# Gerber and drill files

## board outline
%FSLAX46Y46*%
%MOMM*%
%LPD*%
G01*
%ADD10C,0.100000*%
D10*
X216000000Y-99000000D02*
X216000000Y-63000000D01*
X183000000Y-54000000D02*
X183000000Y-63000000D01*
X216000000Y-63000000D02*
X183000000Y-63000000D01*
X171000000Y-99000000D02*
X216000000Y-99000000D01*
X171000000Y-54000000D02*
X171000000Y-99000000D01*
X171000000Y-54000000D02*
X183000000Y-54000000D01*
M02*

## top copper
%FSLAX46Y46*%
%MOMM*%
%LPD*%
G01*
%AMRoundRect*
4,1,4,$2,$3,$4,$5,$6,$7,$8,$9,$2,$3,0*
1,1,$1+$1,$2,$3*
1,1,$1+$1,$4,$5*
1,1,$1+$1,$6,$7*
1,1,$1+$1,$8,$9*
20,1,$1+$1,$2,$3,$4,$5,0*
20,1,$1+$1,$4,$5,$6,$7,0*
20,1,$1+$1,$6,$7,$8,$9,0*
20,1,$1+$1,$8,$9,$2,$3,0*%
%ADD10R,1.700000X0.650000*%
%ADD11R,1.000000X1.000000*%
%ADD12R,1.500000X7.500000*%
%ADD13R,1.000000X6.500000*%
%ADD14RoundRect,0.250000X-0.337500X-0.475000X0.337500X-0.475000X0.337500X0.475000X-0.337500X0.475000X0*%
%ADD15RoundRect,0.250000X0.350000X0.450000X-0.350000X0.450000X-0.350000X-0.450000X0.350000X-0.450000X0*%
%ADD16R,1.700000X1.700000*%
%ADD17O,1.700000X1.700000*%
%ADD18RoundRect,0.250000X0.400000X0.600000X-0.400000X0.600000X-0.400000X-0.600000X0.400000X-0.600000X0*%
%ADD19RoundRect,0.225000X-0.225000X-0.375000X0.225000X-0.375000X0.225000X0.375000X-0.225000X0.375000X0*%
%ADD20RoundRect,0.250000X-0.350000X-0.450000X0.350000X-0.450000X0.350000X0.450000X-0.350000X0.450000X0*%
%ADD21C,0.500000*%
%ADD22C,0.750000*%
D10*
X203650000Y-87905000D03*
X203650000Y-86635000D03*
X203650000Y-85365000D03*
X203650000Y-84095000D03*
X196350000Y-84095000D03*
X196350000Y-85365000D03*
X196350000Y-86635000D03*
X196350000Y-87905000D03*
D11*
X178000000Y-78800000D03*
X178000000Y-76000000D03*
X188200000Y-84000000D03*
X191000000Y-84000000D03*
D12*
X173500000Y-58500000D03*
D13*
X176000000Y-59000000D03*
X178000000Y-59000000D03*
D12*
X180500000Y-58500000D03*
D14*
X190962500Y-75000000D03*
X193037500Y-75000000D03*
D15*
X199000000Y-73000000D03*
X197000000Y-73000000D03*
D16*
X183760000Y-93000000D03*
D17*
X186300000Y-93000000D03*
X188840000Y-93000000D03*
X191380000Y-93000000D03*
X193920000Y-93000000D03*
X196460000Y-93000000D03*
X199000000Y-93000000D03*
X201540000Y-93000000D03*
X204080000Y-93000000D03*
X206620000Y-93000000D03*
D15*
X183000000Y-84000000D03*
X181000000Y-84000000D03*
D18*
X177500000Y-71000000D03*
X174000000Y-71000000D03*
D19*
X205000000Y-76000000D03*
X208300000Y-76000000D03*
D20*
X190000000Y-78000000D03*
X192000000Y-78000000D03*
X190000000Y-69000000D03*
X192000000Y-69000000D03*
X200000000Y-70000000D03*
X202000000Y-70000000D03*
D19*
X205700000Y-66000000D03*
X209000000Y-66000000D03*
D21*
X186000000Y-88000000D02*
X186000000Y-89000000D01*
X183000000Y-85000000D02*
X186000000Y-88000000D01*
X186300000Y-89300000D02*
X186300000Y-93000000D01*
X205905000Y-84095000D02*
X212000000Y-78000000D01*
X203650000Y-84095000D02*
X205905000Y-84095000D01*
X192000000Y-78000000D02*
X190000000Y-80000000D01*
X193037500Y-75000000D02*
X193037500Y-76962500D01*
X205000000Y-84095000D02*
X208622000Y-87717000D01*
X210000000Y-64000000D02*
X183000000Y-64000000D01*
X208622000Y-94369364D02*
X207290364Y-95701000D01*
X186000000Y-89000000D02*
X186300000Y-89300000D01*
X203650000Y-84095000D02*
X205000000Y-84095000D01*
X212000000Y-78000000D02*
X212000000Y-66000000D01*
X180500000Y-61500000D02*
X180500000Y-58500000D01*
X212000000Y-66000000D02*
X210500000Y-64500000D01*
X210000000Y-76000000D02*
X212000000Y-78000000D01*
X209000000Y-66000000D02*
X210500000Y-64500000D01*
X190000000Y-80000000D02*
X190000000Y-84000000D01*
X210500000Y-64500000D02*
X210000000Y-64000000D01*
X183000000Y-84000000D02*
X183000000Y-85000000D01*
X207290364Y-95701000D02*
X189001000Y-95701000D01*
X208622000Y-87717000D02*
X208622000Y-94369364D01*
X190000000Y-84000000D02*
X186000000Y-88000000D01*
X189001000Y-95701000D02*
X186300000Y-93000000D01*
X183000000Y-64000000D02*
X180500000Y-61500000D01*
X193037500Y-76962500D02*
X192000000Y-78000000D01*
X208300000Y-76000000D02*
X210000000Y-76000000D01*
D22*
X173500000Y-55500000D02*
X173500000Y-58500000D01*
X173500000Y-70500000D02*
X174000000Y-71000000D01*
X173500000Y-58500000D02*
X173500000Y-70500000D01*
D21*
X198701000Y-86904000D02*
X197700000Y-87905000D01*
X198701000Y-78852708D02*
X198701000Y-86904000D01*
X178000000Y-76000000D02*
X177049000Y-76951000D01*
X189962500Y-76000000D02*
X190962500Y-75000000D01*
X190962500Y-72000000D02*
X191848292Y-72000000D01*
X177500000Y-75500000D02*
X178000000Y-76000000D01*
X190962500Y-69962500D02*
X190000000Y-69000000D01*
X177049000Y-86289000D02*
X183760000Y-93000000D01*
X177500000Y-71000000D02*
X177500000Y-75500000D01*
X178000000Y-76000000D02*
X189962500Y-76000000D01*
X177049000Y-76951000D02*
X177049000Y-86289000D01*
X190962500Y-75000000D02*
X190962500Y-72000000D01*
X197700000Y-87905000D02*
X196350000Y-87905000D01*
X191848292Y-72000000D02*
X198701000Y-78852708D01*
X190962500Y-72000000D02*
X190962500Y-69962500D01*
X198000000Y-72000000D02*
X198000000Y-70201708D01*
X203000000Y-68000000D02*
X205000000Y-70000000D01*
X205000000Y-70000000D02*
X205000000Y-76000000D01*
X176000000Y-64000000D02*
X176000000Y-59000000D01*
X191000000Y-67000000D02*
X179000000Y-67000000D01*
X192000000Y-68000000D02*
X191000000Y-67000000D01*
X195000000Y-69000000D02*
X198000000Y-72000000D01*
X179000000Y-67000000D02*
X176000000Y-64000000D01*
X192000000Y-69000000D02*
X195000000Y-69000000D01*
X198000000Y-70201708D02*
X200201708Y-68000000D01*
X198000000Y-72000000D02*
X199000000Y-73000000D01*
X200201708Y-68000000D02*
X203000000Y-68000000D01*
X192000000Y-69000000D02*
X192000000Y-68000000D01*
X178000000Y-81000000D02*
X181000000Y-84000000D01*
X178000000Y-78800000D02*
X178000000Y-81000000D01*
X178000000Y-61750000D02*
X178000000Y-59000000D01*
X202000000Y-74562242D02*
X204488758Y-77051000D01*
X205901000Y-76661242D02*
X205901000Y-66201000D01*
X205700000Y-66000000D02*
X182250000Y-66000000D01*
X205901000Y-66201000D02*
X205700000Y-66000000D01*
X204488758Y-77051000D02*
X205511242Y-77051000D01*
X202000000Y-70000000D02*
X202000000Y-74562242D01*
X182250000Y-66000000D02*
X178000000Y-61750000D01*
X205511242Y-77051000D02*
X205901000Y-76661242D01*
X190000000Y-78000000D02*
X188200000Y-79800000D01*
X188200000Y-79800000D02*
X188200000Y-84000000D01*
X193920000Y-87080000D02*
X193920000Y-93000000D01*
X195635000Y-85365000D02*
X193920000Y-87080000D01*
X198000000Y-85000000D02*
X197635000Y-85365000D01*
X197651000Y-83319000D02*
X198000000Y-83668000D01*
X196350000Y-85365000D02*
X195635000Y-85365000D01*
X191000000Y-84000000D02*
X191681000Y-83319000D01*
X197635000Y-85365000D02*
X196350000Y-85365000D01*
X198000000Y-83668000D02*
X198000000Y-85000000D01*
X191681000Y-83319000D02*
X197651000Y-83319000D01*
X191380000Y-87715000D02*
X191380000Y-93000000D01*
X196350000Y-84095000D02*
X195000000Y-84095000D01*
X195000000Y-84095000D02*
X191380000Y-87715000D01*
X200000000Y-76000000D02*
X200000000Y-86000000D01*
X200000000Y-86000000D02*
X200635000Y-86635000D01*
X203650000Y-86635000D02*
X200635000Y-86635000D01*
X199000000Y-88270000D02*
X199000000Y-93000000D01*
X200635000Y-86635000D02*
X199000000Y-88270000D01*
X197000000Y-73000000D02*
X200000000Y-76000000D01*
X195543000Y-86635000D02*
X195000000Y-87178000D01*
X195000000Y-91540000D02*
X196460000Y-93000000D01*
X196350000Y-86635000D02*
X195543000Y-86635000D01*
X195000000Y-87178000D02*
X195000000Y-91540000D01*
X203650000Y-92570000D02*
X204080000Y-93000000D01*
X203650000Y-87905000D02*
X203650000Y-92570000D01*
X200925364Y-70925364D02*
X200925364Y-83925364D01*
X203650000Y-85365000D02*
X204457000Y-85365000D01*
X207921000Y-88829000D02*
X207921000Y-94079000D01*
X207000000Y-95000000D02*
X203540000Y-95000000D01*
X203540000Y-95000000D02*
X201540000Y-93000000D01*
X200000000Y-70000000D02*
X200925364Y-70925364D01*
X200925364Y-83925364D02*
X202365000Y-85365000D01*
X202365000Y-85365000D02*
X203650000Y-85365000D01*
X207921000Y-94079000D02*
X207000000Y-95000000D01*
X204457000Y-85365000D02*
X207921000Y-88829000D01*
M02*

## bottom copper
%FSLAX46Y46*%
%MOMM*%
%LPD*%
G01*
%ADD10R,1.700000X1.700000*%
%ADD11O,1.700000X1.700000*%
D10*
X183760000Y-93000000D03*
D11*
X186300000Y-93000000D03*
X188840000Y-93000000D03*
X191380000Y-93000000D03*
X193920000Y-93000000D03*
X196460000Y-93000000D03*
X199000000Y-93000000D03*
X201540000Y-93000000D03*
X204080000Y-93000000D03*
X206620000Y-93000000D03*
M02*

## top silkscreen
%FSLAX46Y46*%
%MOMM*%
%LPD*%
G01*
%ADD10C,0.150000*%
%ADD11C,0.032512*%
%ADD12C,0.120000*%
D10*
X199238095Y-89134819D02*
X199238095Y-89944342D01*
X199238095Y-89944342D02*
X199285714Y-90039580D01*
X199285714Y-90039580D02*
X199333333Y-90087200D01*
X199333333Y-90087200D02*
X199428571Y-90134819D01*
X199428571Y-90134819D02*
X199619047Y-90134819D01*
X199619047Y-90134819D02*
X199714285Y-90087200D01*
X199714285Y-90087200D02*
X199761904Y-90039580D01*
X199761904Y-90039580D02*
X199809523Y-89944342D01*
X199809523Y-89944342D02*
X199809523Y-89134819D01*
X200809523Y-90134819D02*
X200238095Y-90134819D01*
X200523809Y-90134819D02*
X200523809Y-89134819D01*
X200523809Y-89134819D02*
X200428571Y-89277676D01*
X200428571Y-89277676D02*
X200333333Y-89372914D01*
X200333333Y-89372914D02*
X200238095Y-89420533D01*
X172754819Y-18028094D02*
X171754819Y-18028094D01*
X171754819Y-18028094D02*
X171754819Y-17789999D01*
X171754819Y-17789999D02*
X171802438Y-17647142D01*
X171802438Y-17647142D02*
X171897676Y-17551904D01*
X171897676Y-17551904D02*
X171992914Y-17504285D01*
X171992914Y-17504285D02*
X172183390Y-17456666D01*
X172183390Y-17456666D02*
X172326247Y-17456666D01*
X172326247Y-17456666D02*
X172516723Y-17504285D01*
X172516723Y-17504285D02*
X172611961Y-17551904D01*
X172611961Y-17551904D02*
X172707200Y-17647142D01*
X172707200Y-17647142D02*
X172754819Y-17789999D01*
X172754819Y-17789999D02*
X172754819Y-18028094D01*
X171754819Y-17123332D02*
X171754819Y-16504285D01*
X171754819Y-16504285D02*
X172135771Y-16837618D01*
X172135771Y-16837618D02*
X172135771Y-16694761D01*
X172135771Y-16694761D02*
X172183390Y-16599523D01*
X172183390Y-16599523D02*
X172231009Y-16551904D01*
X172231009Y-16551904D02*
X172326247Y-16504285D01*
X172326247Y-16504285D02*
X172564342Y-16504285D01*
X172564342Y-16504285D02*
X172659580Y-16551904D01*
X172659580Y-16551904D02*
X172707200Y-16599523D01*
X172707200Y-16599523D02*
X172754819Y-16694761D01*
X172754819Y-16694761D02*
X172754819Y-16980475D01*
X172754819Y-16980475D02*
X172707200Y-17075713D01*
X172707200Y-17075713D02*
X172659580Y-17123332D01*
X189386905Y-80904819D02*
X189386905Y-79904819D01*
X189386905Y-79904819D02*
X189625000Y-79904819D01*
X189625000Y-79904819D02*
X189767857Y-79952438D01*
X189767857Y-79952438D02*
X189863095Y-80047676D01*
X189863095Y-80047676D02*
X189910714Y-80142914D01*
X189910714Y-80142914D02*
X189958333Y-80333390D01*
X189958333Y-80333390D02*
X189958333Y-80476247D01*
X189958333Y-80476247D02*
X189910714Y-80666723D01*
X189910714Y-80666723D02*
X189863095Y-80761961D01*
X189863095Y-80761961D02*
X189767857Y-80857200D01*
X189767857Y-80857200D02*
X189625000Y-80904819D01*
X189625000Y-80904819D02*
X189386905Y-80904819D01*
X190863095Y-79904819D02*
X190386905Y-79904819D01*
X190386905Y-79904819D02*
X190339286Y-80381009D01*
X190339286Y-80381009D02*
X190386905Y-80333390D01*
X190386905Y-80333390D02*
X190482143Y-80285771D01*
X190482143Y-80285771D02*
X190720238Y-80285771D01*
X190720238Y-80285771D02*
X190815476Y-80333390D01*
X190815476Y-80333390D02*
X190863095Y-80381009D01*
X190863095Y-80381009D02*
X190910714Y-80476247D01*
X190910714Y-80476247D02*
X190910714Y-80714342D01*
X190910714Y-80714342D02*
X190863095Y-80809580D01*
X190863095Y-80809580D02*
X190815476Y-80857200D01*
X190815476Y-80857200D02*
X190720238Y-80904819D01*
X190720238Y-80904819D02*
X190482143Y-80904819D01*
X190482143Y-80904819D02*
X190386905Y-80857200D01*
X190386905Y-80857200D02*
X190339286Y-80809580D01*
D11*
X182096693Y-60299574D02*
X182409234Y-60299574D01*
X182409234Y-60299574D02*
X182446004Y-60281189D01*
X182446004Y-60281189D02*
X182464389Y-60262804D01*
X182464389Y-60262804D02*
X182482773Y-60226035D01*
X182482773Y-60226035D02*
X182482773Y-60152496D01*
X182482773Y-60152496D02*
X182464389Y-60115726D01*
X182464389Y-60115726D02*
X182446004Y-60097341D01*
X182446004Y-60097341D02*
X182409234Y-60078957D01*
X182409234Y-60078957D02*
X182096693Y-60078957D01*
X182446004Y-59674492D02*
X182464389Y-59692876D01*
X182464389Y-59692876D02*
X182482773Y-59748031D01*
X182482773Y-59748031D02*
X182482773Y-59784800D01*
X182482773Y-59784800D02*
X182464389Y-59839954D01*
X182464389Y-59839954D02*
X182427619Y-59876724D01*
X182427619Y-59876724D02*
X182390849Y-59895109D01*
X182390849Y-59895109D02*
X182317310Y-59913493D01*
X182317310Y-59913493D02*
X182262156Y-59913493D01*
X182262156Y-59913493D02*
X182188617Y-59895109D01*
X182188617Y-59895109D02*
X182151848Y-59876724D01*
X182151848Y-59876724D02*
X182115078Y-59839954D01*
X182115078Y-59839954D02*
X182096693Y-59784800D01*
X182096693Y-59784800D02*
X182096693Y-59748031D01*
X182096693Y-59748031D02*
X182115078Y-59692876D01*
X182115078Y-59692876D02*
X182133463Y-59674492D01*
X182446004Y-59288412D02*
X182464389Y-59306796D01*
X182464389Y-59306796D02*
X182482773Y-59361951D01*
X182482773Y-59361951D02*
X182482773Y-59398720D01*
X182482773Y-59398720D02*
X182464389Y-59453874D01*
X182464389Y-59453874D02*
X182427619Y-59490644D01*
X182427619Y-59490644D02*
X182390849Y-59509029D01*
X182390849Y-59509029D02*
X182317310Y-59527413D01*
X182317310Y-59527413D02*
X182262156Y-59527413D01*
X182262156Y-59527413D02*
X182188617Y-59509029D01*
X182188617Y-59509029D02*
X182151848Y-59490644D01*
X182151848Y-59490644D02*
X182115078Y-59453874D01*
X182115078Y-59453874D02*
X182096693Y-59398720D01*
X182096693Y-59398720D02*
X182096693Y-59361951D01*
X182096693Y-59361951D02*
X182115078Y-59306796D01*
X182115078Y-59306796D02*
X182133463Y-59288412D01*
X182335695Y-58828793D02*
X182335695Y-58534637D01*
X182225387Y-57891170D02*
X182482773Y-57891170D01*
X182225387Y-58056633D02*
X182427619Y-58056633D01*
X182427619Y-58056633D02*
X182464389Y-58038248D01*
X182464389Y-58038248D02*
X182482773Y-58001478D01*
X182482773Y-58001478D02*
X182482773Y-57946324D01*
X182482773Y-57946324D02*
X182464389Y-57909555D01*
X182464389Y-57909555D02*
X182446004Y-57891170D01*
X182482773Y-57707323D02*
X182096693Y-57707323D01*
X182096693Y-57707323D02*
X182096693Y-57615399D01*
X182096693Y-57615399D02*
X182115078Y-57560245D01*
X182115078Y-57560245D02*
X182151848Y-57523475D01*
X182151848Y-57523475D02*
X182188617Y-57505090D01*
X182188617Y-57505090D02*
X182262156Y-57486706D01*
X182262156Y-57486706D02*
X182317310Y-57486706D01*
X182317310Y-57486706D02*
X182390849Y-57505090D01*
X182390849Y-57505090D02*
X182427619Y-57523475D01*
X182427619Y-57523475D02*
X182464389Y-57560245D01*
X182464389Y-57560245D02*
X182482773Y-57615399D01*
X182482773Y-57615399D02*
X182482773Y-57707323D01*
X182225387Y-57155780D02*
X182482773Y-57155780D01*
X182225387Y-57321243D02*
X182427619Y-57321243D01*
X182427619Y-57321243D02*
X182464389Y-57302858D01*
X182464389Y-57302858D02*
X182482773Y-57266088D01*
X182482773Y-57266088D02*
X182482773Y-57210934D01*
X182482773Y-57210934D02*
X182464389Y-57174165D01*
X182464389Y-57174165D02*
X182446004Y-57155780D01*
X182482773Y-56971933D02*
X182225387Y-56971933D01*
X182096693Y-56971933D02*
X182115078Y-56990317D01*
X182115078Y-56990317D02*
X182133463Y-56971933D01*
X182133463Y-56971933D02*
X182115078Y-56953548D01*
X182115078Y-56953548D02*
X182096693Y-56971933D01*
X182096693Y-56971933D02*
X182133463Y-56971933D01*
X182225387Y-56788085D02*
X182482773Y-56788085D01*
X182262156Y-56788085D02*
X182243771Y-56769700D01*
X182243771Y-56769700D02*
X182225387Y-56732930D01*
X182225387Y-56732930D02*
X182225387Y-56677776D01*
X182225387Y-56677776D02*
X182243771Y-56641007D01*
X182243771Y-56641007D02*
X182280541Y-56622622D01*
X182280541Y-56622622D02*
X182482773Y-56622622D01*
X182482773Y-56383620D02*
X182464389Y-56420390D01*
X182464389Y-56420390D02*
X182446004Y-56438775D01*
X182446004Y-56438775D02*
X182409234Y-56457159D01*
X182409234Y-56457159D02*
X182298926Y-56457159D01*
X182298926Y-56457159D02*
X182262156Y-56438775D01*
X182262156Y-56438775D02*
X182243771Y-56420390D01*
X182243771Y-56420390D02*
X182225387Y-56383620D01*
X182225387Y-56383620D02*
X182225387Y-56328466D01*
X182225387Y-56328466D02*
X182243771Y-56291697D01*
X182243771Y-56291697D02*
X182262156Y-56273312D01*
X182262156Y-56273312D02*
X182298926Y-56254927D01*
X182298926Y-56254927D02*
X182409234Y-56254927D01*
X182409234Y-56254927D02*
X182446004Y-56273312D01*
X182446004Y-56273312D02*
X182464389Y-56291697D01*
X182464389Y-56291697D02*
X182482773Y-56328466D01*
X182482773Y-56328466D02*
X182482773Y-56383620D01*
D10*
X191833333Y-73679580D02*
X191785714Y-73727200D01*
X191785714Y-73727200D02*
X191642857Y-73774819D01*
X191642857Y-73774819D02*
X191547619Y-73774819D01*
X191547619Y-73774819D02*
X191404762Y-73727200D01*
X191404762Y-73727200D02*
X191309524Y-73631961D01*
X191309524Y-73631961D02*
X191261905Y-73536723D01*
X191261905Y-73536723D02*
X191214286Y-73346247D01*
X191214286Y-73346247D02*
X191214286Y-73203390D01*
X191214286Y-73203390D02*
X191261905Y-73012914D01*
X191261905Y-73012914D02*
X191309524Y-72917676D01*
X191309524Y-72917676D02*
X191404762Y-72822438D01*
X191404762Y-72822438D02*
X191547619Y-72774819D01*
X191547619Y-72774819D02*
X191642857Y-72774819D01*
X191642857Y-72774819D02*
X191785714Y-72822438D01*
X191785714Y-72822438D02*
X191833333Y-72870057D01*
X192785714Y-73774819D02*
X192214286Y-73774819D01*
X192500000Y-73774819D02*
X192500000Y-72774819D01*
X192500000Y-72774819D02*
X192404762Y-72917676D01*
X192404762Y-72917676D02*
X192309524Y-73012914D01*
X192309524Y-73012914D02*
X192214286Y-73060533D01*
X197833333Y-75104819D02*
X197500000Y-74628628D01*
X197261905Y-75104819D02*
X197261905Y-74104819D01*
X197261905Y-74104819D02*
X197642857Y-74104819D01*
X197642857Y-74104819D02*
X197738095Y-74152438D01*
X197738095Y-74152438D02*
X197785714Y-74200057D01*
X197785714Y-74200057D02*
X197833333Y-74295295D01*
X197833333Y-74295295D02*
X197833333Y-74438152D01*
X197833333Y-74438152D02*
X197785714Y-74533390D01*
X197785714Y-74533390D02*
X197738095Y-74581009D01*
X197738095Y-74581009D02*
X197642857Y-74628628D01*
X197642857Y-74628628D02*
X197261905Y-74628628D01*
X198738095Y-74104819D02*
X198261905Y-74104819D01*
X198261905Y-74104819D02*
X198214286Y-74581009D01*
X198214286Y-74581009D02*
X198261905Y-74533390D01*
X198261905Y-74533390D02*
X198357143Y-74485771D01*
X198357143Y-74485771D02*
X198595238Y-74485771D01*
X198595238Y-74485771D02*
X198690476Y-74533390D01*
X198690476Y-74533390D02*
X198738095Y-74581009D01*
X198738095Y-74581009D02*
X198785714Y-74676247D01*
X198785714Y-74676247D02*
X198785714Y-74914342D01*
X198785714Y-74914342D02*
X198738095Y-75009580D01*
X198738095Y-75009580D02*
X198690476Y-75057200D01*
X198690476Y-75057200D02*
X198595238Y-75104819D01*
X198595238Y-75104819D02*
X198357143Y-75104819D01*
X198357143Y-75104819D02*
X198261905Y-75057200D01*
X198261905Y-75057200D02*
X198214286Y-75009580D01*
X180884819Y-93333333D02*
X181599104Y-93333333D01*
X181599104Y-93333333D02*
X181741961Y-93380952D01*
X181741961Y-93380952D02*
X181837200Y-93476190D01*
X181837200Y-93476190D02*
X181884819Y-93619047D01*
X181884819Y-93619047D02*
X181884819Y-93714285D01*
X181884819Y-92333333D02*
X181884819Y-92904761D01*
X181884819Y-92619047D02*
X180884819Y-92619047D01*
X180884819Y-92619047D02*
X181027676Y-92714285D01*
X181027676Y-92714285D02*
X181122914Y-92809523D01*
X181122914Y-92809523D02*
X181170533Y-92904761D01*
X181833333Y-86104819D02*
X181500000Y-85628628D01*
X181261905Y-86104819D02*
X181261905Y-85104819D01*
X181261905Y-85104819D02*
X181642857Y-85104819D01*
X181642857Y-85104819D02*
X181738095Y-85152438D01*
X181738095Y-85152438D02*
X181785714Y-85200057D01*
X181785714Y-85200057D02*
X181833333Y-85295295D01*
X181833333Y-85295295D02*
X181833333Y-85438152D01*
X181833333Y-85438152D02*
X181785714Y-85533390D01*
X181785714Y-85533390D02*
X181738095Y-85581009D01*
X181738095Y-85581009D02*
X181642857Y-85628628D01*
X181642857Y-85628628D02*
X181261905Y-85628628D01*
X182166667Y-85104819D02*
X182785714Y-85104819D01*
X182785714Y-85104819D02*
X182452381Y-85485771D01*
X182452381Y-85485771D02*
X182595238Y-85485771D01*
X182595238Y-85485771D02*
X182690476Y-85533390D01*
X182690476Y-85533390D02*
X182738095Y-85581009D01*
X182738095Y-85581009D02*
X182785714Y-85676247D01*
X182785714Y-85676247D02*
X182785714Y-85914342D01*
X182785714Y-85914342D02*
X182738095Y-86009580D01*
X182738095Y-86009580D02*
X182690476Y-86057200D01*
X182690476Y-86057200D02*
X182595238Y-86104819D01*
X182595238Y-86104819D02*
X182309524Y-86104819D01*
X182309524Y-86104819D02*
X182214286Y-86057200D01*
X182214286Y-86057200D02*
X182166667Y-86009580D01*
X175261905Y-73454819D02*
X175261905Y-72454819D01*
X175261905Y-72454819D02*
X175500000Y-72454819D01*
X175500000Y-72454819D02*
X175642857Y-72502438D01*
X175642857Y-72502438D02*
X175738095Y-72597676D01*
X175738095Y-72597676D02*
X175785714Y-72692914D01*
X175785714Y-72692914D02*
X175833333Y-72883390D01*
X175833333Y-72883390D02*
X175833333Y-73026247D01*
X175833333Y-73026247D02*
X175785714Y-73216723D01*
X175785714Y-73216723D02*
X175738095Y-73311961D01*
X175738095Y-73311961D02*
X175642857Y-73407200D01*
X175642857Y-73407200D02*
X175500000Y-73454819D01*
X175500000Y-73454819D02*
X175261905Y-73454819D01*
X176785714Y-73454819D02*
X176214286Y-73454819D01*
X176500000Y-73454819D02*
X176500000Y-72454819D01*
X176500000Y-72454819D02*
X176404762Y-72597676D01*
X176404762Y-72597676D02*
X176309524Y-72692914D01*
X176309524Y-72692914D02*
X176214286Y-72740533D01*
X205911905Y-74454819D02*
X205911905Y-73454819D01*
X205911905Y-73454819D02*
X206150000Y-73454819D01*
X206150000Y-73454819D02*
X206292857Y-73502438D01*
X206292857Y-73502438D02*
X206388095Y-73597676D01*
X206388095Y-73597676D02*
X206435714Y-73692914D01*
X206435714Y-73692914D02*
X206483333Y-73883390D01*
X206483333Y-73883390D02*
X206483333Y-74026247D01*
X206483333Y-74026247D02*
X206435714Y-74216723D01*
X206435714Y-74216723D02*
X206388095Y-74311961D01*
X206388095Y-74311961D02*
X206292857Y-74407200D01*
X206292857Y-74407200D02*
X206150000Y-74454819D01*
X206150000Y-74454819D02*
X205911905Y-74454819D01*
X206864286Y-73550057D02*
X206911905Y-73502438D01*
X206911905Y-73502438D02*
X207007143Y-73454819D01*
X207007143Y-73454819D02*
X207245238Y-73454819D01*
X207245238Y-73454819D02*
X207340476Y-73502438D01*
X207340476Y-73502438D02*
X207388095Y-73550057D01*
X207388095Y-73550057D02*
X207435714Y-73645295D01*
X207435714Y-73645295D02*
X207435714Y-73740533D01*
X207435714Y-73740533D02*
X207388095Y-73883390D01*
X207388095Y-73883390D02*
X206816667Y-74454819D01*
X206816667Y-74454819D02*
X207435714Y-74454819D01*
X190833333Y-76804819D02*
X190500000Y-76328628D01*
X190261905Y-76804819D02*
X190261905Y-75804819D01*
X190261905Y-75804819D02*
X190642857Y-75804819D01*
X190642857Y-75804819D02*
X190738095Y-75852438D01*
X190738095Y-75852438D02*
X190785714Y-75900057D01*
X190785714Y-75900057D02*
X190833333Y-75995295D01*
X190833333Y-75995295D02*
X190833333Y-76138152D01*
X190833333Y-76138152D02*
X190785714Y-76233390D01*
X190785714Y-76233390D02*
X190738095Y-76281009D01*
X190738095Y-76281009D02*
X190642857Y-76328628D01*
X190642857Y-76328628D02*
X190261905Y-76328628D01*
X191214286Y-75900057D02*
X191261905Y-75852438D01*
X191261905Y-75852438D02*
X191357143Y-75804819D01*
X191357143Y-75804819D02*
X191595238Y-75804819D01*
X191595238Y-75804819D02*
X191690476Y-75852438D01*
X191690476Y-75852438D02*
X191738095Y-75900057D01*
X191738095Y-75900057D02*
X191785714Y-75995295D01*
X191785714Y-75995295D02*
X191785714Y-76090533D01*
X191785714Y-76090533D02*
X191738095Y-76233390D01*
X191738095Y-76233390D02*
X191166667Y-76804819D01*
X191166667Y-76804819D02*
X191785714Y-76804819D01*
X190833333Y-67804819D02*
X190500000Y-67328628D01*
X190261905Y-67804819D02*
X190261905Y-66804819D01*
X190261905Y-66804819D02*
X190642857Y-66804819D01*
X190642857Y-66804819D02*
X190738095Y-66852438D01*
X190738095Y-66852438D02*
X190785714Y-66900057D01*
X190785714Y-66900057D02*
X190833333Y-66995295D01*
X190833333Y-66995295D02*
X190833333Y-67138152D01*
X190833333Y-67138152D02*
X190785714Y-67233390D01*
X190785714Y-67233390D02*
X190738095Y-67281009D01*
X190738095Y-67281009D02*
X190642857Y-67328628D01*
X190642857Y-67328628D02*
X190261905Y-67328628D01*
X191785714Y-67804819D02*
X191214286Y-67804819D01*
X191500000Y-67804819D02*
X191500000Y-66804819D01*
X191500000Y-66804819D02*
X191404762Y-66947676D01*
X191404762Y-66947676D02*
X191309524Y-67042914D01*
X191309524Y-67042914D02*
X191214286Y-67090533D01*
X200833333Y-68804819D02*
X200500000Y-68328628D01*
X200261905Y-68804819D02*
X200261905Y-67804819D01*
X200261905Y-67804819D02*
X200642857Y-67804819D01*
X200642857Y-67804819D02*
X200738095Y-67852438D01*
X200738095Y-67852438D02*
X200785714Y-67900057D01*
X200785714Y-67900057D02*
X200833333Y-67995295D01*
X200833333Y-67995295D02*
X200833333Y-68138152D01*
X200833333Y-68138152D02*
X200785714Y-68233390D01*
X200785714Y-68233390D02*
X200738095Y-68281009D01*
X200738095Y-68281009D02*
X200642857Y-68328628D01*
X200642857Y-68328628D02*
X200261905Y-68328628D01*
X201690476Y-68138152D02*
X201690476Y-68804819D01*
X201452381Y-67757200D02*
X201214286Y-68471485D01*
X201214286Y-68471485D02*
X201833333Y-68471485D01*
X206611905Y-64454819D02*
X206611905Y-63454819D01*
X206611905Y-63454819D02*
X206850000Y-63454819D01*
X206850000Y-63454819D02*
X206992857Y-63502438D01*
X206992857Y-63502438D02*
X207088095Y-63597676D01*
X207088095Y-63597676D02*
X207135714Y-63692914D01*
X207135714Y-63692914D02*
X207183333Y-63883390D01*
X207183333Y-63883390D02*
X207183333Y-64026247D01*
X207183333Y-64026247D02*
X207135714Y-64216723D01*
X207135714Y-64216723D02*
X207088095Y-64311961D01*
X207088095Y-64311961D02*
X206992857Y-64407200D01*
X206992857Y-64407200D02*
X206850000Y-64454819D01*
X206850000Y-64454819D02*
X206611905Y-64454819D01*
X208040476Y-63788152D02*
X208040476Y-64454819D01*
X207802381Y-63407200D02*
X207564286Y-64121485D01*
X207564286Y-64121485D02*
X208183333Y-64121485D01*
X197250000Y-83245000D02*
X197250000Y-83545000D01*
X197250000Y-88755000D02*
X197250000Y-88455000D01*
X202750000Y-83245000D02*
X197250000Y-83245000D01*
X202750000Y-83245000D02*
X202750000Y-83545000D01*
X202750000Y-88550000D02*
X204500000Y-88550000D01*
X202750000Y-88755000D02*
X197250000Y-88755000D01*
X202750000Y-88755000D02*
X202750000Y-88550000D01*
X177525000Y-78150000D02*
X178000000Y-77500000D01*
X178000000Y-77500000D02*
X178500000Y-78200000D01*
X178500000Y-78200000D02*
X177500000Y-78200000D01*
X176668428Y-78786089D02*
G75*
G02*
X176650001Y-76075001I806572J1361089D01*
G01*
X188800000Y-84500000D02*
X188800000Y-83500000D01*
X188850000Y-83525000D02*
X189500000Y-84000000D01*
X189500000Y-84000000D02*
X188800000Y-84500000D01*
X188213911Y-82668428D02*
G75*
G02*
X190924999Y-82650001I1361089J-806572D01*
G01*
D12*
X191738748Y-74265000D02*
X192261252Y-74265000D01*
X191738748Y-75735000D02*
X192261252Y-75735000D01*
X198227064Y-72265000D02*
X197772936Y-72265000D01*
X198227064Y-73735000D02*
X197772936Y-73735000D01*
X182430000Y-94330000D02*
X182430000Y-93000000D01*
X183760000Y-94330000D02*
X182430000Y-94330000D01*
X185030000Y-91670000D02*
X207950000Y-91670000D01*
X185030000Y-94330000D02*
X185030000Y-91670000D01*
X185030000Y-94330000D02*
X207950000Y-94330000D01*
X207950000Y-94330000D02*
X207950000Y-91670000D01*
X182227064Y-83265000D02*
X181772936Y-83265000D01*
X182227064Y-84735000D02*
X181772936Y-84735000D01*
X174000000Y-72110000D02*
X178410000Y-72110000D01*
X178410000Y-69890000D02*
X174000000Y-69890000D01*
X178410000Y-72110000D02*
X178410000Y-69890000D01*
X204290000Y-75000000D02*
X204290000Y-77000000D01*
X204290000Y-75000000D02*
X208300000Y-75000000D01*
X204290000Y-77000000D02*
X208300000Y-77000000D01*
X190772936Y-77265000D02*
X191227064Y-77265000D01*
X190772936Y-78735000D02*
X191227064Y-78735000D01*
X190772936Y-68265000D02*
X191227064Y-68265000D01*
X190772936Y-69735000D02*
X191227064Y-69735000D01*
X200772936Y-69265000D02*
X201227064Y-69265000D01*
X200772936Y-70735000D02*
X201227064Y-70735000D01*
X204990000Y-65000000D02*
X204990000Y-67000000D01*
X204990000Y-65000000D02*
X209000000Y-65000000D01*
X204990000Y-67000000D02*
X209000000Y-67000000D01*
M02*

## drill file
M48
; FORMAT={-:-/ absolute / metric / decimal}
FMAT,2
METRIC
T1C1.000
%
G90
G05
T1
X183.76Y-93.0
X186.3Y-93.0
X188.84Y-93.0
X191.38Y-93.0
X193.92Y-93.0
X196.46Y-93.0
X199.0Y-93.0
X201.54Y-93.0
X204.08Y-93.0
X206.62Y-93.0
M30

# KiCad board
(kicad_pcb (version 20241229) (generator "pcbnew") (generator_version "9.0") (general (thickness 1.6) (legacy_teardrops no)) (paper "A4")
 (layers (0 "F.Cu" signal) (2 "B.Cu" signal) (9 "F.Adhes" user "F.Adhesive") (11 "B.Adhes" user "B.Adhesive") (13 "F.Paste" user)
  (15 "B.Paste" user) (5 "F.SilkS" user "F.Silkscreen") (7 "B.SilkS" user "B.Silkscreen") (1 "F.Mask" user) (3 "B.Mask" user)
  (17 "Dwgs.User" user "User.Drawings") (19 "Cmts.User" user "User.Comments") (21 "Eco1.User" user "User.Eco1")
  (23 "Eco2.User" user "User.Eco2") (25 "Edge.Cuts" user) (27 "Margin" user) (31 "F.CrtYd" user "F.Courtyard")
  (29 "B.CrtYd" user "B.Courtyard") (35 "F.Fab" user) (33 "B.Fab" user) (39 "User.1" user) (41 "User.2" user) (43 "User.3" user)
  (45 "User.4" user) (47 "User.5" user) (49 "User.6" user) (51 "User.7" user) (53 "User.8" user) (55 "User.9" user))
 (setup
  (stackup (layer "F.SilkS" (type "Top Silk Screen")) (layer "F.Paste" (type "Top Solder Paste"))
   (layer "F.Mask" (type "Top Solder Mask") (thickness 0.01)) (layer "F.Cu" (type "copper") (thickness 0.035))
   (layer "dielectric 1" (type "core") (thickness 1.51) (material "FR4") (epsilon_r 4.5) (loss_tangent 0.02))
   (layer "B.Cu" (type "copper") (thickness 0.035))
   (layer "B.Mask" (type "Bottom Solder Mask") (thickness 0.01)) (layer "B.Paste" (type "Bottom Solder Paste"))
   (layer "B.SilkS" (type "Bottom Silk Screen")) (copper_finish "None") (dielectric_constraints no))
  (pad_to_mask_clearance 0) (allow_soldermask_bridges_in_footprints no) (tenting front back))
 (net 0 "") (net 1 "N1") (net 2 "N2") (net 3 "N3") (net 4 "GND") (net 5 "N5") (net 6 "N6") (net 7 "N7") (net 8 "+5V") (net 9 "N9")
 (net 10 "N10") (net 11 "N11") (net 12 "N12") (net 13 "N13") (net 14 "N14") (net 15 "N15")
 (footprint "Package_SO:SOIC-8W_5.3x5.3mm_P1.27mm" (layer "F.Cu") (at 200 86 180)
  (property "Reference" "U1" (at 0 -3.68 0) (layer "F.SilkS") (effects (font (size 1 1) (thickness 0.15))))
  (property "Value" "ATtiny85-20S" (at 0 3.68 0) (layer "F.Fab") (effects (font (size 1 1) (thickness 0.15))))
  (fp_line (start 2.75 2.755) (end 2.75 2.455) (stroke (width 0.15) (type solid)) (layer "F.SilkS"))
  (fp_line (start 2.75 -2.755) (end 2.75 -2.455) (stroke (width 0.15) (type solid)) (layer "F.SilkS"))
  (fp_line (start -2.75 2.755) (end 2.75 2.755) (stroke (width 0.15) (type solid)) (layer "F.SilkS"))
  (fp_line (start -2.75 2.755) (end -2.75 2.455) (stroke (width 0.15) (type solid)) (layer "F.SilkS"))
  (fp_line (start -2.75 -2.55) (end -4.5 -2.55) (stroke (width 0.15) (type solid)) (layer "F.SilkS"))
  (fp_line (start -2.75 -2.755) (end 2.75 -2.755) (stroke (width 0.15) (type solid)) (layer "F.SilkS"))
  (fp_line (start -2.75 -2.755) (end -2.75 -2.55) (stroke (width 0.15) (type solid)) (layer "F.SilkS"))
  (pad "1" smd rect (at -3.65 -1.905 180) (size 1.7 0.65) (layers "F.Cu" "F.Mask" "F.Paste") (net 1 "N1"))
  (pad "2" smd rect (at -3.65 -0.635 180) (size 1.7 0.65) (layers "F.Cu" "F.Mask" "F.Paste") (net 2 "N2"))
  (pad "3" smd rect (at -3.65 0.635 180) (size 1.7 0.65) (layers "F.Cu" "F.Mask" "F.Paste") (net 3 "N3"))
  (pad "4" smd rect (at -3.65 1.905 180) (size 1.7 0.65) (layers "F.Cu" "F.Mask" "F.Paste") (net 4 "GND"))
  (pad "5" smd rect (at 3.65 1.905 180) (size 1.7 0.65) (layers "F.Cu" "F.Mask" "F.Paste") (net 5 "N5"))
  (pad "6" smd rect (at 3.65 0.635 180) (size 1.7 0.65) (layers "F.Cu" "F.Mask" "F.Paste") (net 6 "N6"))
  (pad "7" smd rect (at 3.65 -0.635 180) (size 1.7 0.65) (layers "F.Cu" "F.Mask" "F.Paste") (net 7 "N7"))
  (pad "8" smd rect (at 3.65 -1.905 180) (size 1.7 0.65) (layers "F.Cu" "F.Mask" "F.Paste") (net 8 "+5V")))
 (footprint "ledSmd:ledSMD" (layer "F.Cu") (at 178 77 90)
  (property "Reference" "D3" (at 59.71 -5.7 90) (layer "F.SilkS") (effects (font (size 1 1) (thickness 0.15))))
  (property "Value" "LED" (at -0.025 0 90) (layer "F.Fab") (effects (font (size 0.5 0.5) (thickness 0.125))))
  (fp_line (start -1.15 -0.475) (end -0.5 0) (stroke (width 0.15) (type solid)) (layer "F.SilkS"))
  (fp_line (start -0.5 0) (end -1.2 0.5) (stroke (width 0.15) (type solid)) (layer "F.SilkS"))
  (fp_line (start -1.2 0.5) (end -1.2 -0.5) (stroke (width 0.15) (type solid)) (layer "F.SilkS"))
  (fp_arc (start -1.786089 -1.331572) (mid -0.435753 -2.107089) (end 0.924999 -1.349999) (stroke (width 0.15) (type solid))
   (layer "F.SilkS"))
  (pad "1" smd rect (at -1.8 0 90) (size 1 1) (layers "F.Cu" "F.Mask" "F.Paste") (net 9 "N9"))
  (pad "2" smd rect (at 1 0 90) (size 1 1) (layers "F.Cu" "F.Mask" "F.Paste") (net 8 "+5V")))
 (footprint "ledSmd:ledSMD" (layer "F.Cu") (at 190 84)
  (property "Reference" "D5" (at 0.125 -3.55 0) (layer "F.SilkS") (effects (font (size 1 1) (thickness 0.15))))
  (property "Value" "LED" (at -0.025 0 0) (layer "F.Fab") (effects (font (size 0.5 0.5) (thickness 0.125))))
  (fp_line (start -1.2 0.5) (end -1.2 -0.5) (stroke (width 0.15) (type solid)) (layer "F.SilkS"))
  (fp_line (start -1.15 -0.475) (end -0.5 0) (stroke (width 0.15) (type solid)) (layer "F.SilkS"))
  (fp_line (start -0.5 0) (end -1.2 0.5) (stroke (width 0.15) (type solid)) (layer "F.SilkS"))
  (fp_arc (start -1.786089 -1.331572) (mid -0.435753 -2.107089) (end 0.924999 -1.349999) (stroke (width 0.15) (type solid))
   (layer "F.SilkS"))
  (pad "1" smd rect (at -1.8 0) (size 1 1) (layers "F.Cu" "F.Mask" "F.Paste") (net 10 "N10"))
  (pad "2" smd rect (at 1 0) (size 1 1) (layers "F.Cu" "F.Mask" "F.Paste") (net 6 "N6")))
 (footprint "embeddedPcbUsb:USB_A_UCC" (layer "F.Cu") (at 177 58.7 -90)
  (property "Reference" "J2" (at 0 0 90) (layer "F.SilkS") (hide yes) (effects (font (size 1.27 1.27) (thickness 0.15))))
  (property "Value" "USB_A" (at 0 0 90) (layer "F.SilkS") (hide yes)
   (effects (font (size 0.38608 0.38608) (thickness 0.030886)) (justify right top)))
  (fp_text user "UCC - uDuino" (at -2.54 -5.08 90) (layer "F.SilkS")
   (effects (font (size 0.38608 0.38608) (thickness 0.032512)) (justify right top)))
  (pad "1" smd rect (at -0.2 3.5 270) (size 7.5 1.5) (layers "F.Cu" "F.Mask" "F.Paste") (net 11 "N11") (solder_mask_margin 0.1016))
  (pad "2" smd rect (at 0.3 1 270) (size 6.5 1) (layers "F.Cu" "F.Mask" "F.Paste") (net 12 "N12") (solder_mask_margin 0.1016))
  (pad "3" smd rect (at 0.3 -1 270) (size 6.5 1) (layers "F.Cu" "F.Mask" "F.Paste") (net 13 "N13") (solder_mask_margin 0.1016))
  (pad "4" smd rect (at -0.2 -3.5 270) (size 7.5 1.5) (layers "F.Cu" "F.Mask" "F.Paste") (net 4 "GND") (solder_mask_margin 0.1016)))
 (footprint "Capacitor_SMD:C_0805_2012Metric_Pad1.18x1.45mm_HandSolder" (layer "F.Cu") (at 192 75)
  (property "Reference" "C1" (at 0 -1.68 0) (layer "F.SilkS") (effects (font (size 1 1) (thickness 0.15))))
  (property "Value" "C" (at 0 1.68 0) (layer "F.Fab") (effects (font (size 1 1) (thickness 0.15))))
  (fp_line (start -0.261252 -0.735) (end 0.261252 -0.735) (stroke (width 0.12) (type solid)) (layer "F.SilkS"))
  (fp_line (start -0.261252 0.735) (end 0.261252 0.735) (stroke (width 0.12) (type solid)) (layer "F.SilkS"))
  (pad "1" smd roundrect (at -1.0375 0) (size 1.175 1.45) (layers "F.Cu" "F.Mask" "F.Paste") (roundrect_rratio 0.212766) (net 8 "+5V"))
  (pad "2" smd roundrect (at 1.0375 0) (size 1.175 1.45) (layers "F.Cu" "F.Mask" "F.Paste") (roundrect_rratio 0.212766) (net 4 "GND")))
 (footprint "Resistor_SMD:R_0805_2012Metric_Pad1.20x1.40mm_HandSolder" (layer "F.Cu") (at 198 73 180)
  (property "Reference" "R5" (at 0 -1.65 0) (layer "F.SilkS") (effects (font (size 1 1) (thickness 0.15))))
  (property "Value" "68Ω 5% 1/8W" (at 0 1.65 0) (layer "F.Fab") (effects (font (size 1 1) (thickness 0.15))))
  (fp_line (start -0.227064 0.735) (end 0.227064 0.735) (stroke (width 0.12) (type solid)) (layer "F.SilkS"))
  (fp_line (start -0.227064 -0.735) (end 0.227064 -0.735) (stroke (width 0.12) (type solid)) (layer "F.SilkS"))
  (pad "1" smd roundrect (at -1 0 180) (size 1.2 1.4) (layers "F.Cu" "F.Mask" "F.Paste") (roundrect_rratio 0.208333) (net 12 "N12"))
  (pad "2" smd roundrect (at 1 0 180) (size 1.2 1.4) (layers "F.Cu" "F.Mask" "F.Paste") (roundrect_rratio 0.208333) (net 2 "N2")))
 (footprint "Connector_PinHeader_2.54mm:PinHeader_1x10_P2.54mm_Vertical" (layer "F.Cu") (at 183.76 93 90)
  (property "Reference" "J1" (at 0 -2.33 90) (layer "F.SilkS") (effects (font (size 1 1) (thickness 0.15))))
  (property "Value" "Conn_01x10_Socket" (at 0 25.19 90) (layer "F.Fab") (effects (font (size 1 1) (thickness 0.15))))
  (fp_line (start -1.33 -1.33) (end 0 -1.33) (stroke (width 0.12) (type solid)) (layer "F.SilkS"))
  (fp_line (start -1.33 0) (end -1.33 -1.33) (stroke (width 0.12) (type solid)) (layer "F.SilkS"))
  (fp_line (start 1.33 1.27) (end 1.33 24.19) (stroke (width 0.12) (type solid)) (layer "F.SilkS"))
  (fp_line (start -1.33 1.27) (end 1.33 1.27) (stroke (width 0.12) (type solid)) (layer "F.SilkS"))
  (fp_line (start -1.33 1.27) (end -1.33 24.19) (stroke (width 0.12) (type solid)) (layer "F.SilkS"))
  (fp_line (start -1.33 24.19) (end 1.33 24.19) (stroke (width 0.12) (type solid)) (layer "F.SilkS"))
  (pad "1" thru_hole rect (at 0 0 90) (size 1.7 1.7) (drill 1) (layers "*.Cu" "*.Mask") (remove_unused_layers no) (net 8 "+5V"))
  (pad "2" thru_hole oval (at 0 2.54 90) (size 1.7 1.7) (drill 1) (layers "*.Cu" "*.Mask") (remove_unused_layers no) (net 4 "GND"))
  (pad "3" thru_hole oval (at 0 5.08 90) (size 1.7 1.7) (drill 1) (layers "*.Cu" "*.Mask") (remove_unused_layers no) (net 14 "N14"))
  (pad "4" thru_hole oval (at 0 7.62 90) (size 1.7 1.7) (drill 1) (layers "*.Cu" "*.Mask") (remove_unused_layers no) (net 5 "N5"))
  (pad "5" thru_hole oval (at 0 10.16 90) (size 1.7 1.7) (drill 1) (layers "*.Cu" "*.Mask") (remove_unused_layers no) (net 6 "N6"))
  (pad "6" thru_hole oval (at 0 12.7 90) (size 1.7 1.7) (drill 1) (layers "*.Cu" "*.Mask") (remove_unused_layers no) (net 7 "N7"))
  (pad "7" thru_hole oval (at 0 15.24 90) (size 1.7 1.7) (drill 1) (layers "*.Cu" "*.Mask") (remove_unused_layers no) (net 2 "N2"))
  (pad "8" thru_hole oval (at 0 17.78 90) (size 1.7 1.7) (drill 1) (layers "*.Cu" "*.Mask") (remove_unused_layers no) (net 3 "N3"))
  (pad "9" thru_hole oval (at 0 20.32 90) (size 1.7 1.7) (drill 1) (layers "*.Cu" "*.Mask") (remove_unused_layers no) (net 1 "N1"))
  (pad "10" thru_hole oval (at 0 22.86 90) (size 1.7 1.7) (drill 1) (layers "*.Cu" "*.Mask") (remove_unused_layers no) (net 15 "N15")))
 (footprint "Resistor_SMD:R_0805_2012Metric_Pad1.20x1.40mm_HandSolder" (layer "F.Cu") (at 182 84 180)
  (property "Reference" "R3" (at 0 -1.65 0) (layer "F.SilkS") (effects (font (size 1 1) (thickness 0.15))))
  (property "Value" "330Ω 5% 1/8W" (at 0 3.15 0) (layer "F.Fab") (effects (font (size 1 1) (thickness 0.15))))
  (fp_line (start -0.227064 0.735) (end 0.227064 0.735) (stroke (width 0.12) (type solid)) (layer "F.SilkS"))
  (fp_line (start -0.227064 -0.735) (end 0.227064 -0.735) (stroke (width 0.12) (type solid)) (layer "F.SilkS"))
  (pad "1" smd roundrect (at -1 0 180) (size 1.2 1.4) (layers "F.Cu" "F.Mask" "F.Paste") (roundrect_rratio 0.208333) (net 4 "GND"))
  (pad "2" smd roundrect (at 1 0 180) (size 1.2 1.4) (layers "F.Cu" "F.Mask" "F.Paste") (roundrect_rratio 0.208333) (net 9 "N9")))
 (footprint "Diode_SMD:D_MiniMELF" (layer "F.Cu") (at 175.75 71 180)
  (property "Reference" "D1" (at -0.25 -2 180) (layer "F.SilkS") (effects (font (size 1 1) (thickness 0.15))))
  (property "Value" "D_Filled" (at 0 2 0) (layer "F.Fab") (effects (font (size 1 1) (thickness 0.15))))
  (fp_line (start 1.75 -1.11) (end -2.66 -1.11) (stroke (width 0.12) (type solid)) (layer "F.SilkS"))
  (fp_line (start -2.66 1.11) (end 1.75 1.11) (stroke (width 0.12) (type solid)) (layer "F.SilkS"))
  (fp_line (start -2.66 -1.11) (end -2.66 1.11) (stroke (width 0.12) (type solid)) (layer "F.SilkS"))
  (pad "1" smd roundrect (at -1.75 0 180) (size 1.3 1.7) (layers "F.Cu" "F.Mask" "F.Paste") (roundrect_rratio 0.1923076923) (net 8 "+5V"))
  (pad "2" smd roundrect (at 1.75 0 180) (size 1.3 1.7) (layers "F.Cu" "F.Mask" "F.Paste") (roundrect_rratio 0.1923076923) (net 11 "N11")))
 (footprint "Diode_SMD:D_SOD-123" (layer "F.Cu") (at 206.65 76)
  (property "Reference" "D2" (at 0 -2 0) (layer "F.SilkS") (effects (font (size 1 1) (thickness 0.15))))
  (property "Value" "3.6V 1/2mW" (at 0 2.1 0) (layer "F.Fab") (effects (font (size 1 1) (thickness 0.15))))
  (fp_line (start -2.36 -1) (end -2.36 1) (stroke (width 0.12) (type solid)) (layer "F.SilkS"))
  (fp_line (start -2.36 -1) (end 1.65 -1) (stroke (width 0.12) (type solid)) (layer "F.SilkS"))
  (fp_line (start -2.36 1) (end 1.65 1) (stroke (width 0.12) (type solid)) (layer "F.SilkS"))
  (pad "1" smd roundrect (at -1.65 0) (size 0.9 1.2) (layers "F.Cu" "F.Mask" "F.Paste") (roundrect_rratio 0.25) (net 12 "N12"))
  (pad "2" smd roundrect (at 1.65 0) (size 0.9 1.2) (layers "F.Cu" "F.Mask" "F.Paste") (roundrect_rratio 0.25) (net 4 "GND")))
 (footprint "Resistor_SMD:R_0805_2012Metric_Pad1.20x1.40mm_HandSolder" (layer "F.Cu") (at 191 78)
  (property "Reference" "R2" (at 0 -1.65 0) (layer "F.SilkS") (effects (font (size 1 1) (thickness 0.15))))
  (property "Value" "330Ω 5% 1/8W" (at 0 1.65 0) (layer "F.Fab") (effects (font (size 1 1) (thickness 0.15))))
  (fp_line (start -0.227064 -0.735) (end 0.227064 -0.735) (stroke (width 0.12) (type solid)) (layer "F.SilkS"))
  (fp_line (start -0.227064 0.735) (end 0.227064 0.735) (stroke (width 0.12) (type solid)) (layer "F.SilkS"))
  (pad "1" smd roundrect (at -1 0) (size 1.2 1.4) (layers "F.Cu" "F.Mask" "F.Paste") (roundrect_rratio 0.208333) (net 10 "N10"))
  (pad "2" smd roundrect (at 1 0) (size 1.2 1.4) (layers "F.Cu" "F.Mask" "F.Paste") (roundrect_rratio 0.208333) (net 4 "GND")))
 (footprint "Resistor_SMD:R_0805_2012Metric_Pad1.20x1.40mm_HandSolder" (layer "F.Cu") (at 191 69)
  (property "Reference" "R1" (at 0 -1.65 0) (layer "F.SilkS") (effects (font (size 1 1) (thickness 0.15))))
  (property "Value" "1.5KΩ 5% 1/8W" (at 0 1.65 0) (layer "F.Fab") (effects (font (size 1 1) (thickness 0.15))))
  (fp_line (start -0.227064 -0.735) (end 0.227064 -0.735) (stroke (width 0.12) (type solid)) (layer "F.SilkS"))
  (fp_line (start -0.227064 0.735) (end 0.227064 0.735) (stroke (width 0.12) (type solid)) (layer "F.SilkS"))
  (pad "1" smd roundrect (at -1 0) (size 1.2 1.4) (layers "F.Cu" "F.Mask" "F.Paste") (roundrect_rratio 0.208333) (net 8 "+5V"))
  (pad "2" smd roundrect (at 1 0) (size 1.2 1.4) (layers "F.Cu" "F.Mask" "F.Paste") (roundrect_rratio 0.208333) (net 12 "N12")))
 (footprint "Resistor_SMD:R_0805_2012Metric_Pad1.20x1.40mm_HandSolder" (layer "F.Cu") (at 201 70)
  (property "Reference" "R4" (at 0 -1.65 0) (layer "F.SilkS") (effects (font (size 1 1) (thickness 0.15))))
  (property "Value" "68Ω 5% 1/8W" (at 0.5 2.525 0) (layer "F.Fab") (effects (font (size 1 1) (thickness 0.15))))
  (fp_line (start -0.227064 -0.735) (end 0.227064 -0.735) (stroke (width 0.12) (type solid)) (layer "F.SilkS"))
  (fp_line (start -0.227064 0.735) (end 0.227064 0.735) (stroke (width 0.12) (type solid)) (layer "F.SilkS"))
  (pad "1" smd roundrect (at -1 0) (size 1.2 1.4) (layers "F.Cu" "F.Mask" "F.Paste") (roundrect_rratio 0.208333) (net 3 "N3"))
  (pad "2" smd roundrect (at 1 0) (size 1.2 1.4) (layers "F.Cu" "F.Mask" "F.Paste") (roundrect_rratio 0.208333) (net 13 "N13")))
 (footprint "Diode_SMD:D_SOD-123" (layer "F.Cu") (at 207.35 66)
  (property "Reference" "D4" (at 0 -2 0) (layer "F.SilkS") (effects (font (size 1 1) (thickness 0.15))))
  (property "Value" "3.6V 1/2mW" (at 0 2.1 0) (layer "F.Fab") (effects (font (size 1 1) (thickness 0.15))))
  (fp_line (start -2.36 -1) (end -2.36 1) (stroke (width 0.12) (type solid)) (layer "F.SilkS"))
  (fp_line (start -2.36 -1) (end 1.65 -1) (stroke (width 0.12) (type solid)) (layer "F.SilkS"))
  (fp_line (start -2.36 1) (end 1.65 1) (stroke (width 0.12) (type solid)) (layer "F.SilkS"))
  (pad "1" smd roundrect (at -1.65 0) (size 0.9 1.2) (layers "F.Cu" "F.Mask" "F.Paste") (roundrect_rratio 0.25) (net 13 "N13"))
  (pad "2" smd roundrect (at 1.65 0) (size 0.9 1.2) (layers "F.Cu" "F.Mask" "F.Paste") (roundrect_rratio 0.25) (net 4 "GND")))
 (gr_line (start 216 99) (end 216 63) (stroke (width 0.1) (type default)) (layer "Edge.Cuts"))
 (gr_line (start 183 54) (end 183 63) (stroke (width 0.1) (type default)) (layer "Edge.Cuts"))
 (gr_line (start 216 63) (end 183 63) (stroke (width 0.1) (type default)) (layer "Edge.Cuts"))
 (gr_line (start 171 99) (end 216 99) (stroke (width 0.1) (type default)) (layer "Edge.Cuts"))
 (gr_line (start 171 54) (end 171 99) (stroke (width 0.1) (type default)) (layer "Edge.Cuts"))
 (gr_line (start 171 54) (end 183 54) (stroke (width 0.1) (type default)) (layer "Edge.Cuts"))
 (segment (start 186 88) (end 186 89) (width 0.5) (layer "F.Cu") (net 4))
 (segment (start 183 85) (end 186 88) (width 0.5) (layer "F.Cu") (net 4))
 (segment (start 186.3 89.3) (end 186.3 93) (width 0.5) (layer "F.Cu") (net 4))
 (segment (start 205.905 84.095) (end 212 78) (width 0.5) (layer "F.Cu") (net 4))
 (segment (start 203.65 84.095) (end 205.905 84.095) (width 0.5) (layer "F.Cu") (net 4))
 (segment (start 192 78) (end 190 80) (width 0.5) (layer "F.Cu") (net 4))
 (segment (start 193.0375 75) (end 193.0375 76.9625) (width 0.5) (layer "F.Cu") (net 4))
 (segment (start 205 84.095) (end 208.622 87.717) (width 0.5) (layer "F.Cu") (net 4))
 (segment (start 210 64) (end 183 64) (width 0.5) (layer "F.Cu") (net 4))
 (segment (start 208.622 94.369364) (end 207.290364 95.701) (width 0.5) (layer "F.Cu") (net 4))
 (segment (start 186 89) (end 186.3 89.3) (width 0.5) (layer "F.Cu") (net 4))
 (segment (start 203.65 84.095) (end 205 84.095) (width 0.5) (layer "F.Cu") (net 4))
 (segment (start 212 78) (end 212 66) (width 0.5) (layer "F.Cu") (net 4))
 (segment (start 180.5 61.5) (end 180.5 58.5) (width 0.5) (layer "F.Cu") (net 4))
 (segment (start 212 66) (end 210.5 64.5) (width 0.5) (layer "F.Cu") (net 4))
 (segment (start 210 76) (end 212 78) (width 0.5) (layer "F.Cu") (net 4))
 (segment (start 209 66) (end 210.5 64.5) (width 0.5) (layer "F.Cu") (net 4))
 (segment (start 190 80) (end 190 84) (width 0.5) (layer "F.Cu") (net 4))
 (segment (start 210.5 64.5) (end 210 64) (width 0.5) (layer "F.Cu") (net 4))
 (segment (start 183 84) (end 183 85) (width 0.5) (layer "F.Cu") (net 4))
 (segment (start 207.290364 95.701) (end 189.001 95.701) (width 0.5) (layer "F.Cu") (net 4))
 (segment (start 208.622 87.717) (end 208.622 94.369364) (width 0.5) (layer "F.Cu") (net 4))
 (segment (start 190 84) (end 186 88) (width 0.5) (layer "F.Cu") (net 4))
 (segment (start 189.001 95.701) (end 186.3 93) (width 0.5) (layer "F.Cu") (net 4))
 (segment (start 183 64) (end 180.5 61.5) (width 0.5) (layer "F.Cu") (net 4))
 (segment (start 193.0375 76.9625) (end 192 78) (width 0.5) (layer "F.Cu") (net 4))
 (segment (start 208.3 76) (end 210 76) (width 0.5) (layer "F.Cu") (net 4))
 (segment (start 173.5 55.5) (end 173.5 58.5) (width 0.75) (layer "F.Cu") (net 11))
 (segment (start 173.5 70.5) (end 174 71) (width 0.75) (layer "F.Cu") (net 11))
 (segment (start 173.5 58.5) (end 173.5 70.5) (width 0.75) (layer "F.Cu") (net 11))
 (segment (start 198.701 86.904) (end 197.7 87.905) (width 0.5) (layer "F.Cu") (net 8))
 (segment (start 198.701 78.852708) (end 198.701 86.904) (width 0.5) (layer "F.Cu") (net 8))
 (segment (start 178 76) (end 177.049 76.951) (width 0.5) (layer "F.Cu") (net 8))
 (segment (start 189.9625 76) (end 190.9625 75) (width 0.5) (layer "F.Cu") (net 8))
 (segment (start 190.9625 72) (end 191.848292 72) (width 0.5) (layer "F.Cu") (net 8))
 (segment (start 177.5 75.5) (end 178 76) (width 0.5) (layer "F.Cu") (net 8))
 (segment (start 190.9625 69.9625) (end 190 69) (width 0.5) (layer "F.Cu") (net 8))
 (segment (start 177.049 86.289) (end 183.76 93) (width 0.5) (layer "F.Cu") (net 8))
 (segment (start 177.5 71) (end 177.5 75.5) (width 0.5) (layer "F.Cu") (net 8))
 (segment (start 178 76) (end 189.9625 76) (width 0.5) (layer "F.Cu") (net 8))
 (segment (start 177.049 76.951) (end 177.049 86.289) (width 0.5) (layer "F.Cu") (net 8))
 (segment (start 190.9625 75) (end 190.9625 72) (width 0.5) (layer "F.Cu") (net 8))
 (segment (start 197.7 87.905) (end 196.35 87.905) (width 0.5) (layer "F.Cu") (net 8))
 (segment (start 191.848292 72) (end 198.701 78.852708) (width 0.5) (layer "F.Cu") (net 8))
 (segment (start 190.9625 72) (end 190.9625 69.9625) (width 0.5) (layer "F.Cu") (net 8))
 (segment (start 198 72) (end 198 70.201708) (width 0.5) (layer "F.Cu") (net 12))
 (segment (start 203 68) (end 205 70) (width 0.5) (layer "F.Cu") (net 12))
 (segment (start 205 70) (end 205 76) (width 0.5) (layer "F.Cu") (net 12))
 (segment (start 176 64) (end 176 59) (width 0.5) (layer "F.Cu") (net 12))
 (segment (start 191 67) (end 179 67) (width 0.5) (layer "F.Cu") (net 12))
 (segment (start 192 68) (end 191 67) (width 0.5) (layer "F.Cu") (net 12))
 (segment (start 195 69) (end 198 72) (width 0.5) (layer "F.Cu") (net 12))
 (segment (start 179 67) (end 176 64) (width 0.5) (layer "F.Cu") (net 12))
 (segment (start 192 69) (end 195 69) (width 0.5) (layer "F.Cu") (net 12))
 (segment (start 198 70.201708) (end 200.201708 68) (width 0.5) (layer "F.Cu") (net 12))
 (segment (start 198 72) (end 199 73) (width 0.5) (layer "F.Cu") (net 12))
 (segment (start 200.201708 68) (end 203 68) (width 0.5) (layer "F.Cu") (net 12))
 (segment (start 192 69) (end 192 68) (width 0.5) (layer "F.Cu") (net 12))
 (segment (start 178 81) (end 181 84) (width 0.5) (layer "F.Cu") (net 9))
 (segment (start 178 78.8) (end 178 81) (width 0.5) (layer "F.Cu") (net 9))
 (segment (start 178 61.75) (end 178 59) (width 0.5) (layer "F.Cu") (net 13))
 (segment (start 202 74.562242) (end 204.488758 77.051) (width 0.5) (layer "F.Cu") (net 13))
 (segment (start 205.901 76.661242) (end 205.901 66.201) (width 0.5) (layer "F.Cu") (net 13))
 (segment (start 205.7 66) (end 182.25 66) (width 0.5) (layer "F.Cu") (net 13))
 (segment (start 205.901 66.201) (end 205.7 66) (width 0.5) (layer "F.Cu") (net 13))
 (segment (start 204.488758 77.051) (end 205.511242 77.051) (width 0.5) (layer "F.Cu") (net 13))
 (segment (start 202 70) (end 202 74.562242) (width 0.5) (layer "F.Cu") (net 13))
 (segment (start 182.25 66) (end 178 61.75) (width 0.5) (layer "F.Cu") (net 13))
 (segment (start 205.511242 77.051) (end 205.901 76.661242) (width 0.5) (layer "F.Cu") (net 13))
 (segment (start 190 78) (end 188.2 79.8) (width 0.5) (layer "F.Cu") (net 10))
 (segment (start 188.2 79.8) (end 188.2 84) (width 0.5) (layer "F.Cu") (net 10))
 (segment (start 193.92 87.08) (end 193.92 93) (width 0.5) (layer "F.Cu") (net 6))
 (segment (start 195.635 85.365) (end 193.92 87.08) (width 0.5) (layer "F.Cu") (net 6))
 (segment (start 198 85) (end 197.635 85.365) (width 0.5) (layer "F.Cu") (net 6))
 (segment (start 197.651 83.319) (end 198 83.668) (width 0.5) (layer "F.Cu") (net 6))
 (segment (start 196.35 85.365) (end 195.635 85.365) (width 0.5) (layer "F.Cu") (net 6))
 (segment (start 191 84) (end 191.681 83.319) (width 0.5) (layer "F.Cu") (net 6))
 (segment (start 197.635 85.365) (end 196.35 85.365) (width 0.5) (layer "F.Cu") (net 6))
 (segment (start 198 83.668) (end 198 85) (width 0.5) (layer "F.Cu") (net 6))
 (segment (start 191.681 83.319) (end 197.651 83.319) (width 0.5) (layer "F.Cu") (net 6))
 (segment (start 191.38 87.715) (end 191.38 93) (width 0.5) (layer "F.Cu") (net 5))
 (segment (start 196.35 84.095) (end 195 84.095) (width 0.5) (layer "F.Cu") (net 5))
 (segment (start 195 84.095) (end 191.38 87.715) (width 0.5) (layer "F.Cu") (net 5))
 (segment (start 200 76) (end 200 86) (width 0.5) (layer "F.Cu") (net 2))
 (segment (start 200 86) (end 200.635 86.635) (width 0.5) (layer "F.Cu") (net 2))
 (segment (start 203.65 86.635) (end 200.635 86.635) (width 0.5) (layer "F.Cu") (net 2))
 (segment (start 199 88.27) (end 199 93) (width 0.5) (layer "F.Cu") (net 2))
 (segment (start 200.635 86.635) (end 199 88.27) (width 0.5) (layer "F.Cu") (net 2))
 (segment (start 197 73) (end 200 76) (width 0.5) (layer "F.Cu") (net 2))
 (segment (start 195.543 86.635) (end 195 87.178) (width 0.5) (layer "F.Cu") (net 7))
 (segment (start 195 91.54) (end 196.46 93) (width 0.5) (layer "F.Cu") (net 7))
 (segment (start 196.35 86.635) (end 195.543 86.635) (width 0.5) (layer "F.Cu") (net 7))
 (segment (start 195 87.178) (end 195 91.54) (width 0.5) (layer "F.Cu") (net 7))
 (segment (start 203.65 92.57) (end 204.08 93) (width 0.5) (layer "F.Cu") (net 1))
 (segment (start 203.65 87.905) (end 203.65 92.57) (width 0.5) (layer "F.Cu") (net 1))
 (segment (start 200.925364 70.925364) (end 200.925364 83.925364) (width 0.5) (layer "F.Cu") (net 3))
 (segment (start 203.65 85.365) (end 204.457 85.365) (width 0.5) (layer "F.Cu") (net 3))
 (segment (start 207.921 88.829) (end 207.921 94.079) (width 0.5) (layer "F.Cu") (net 3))
 (segment (start 207 95) (end 203.54 95) (width 0.5) (layer "F.Cu") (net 3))
 (segment (start 203.54 95) (end 201.54 93) (width 0.5) (layer "F.Cu") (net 3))
 (segment (start 200 70) (end 200.925364 70.925364) (width 0.5) (layer "F.Cu") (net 3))
 (segment (start 200.925364 83.925364) (end 202.365 85.365) (width 0.5) (layer "F.Cu") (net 3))
 (segment (start 202.365 85.365) (end 203.65 85.365) (width 0.5) (layer "F.Cu") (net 3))
 (segment (start 207.921 94.079) (end 207 95) (width 0.5) (layer "F.Cu") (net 3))
 (segment (start 204.457 85.365) (end 207.921 88.829) (width 0.5) (layer "F.Cu") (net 3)))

